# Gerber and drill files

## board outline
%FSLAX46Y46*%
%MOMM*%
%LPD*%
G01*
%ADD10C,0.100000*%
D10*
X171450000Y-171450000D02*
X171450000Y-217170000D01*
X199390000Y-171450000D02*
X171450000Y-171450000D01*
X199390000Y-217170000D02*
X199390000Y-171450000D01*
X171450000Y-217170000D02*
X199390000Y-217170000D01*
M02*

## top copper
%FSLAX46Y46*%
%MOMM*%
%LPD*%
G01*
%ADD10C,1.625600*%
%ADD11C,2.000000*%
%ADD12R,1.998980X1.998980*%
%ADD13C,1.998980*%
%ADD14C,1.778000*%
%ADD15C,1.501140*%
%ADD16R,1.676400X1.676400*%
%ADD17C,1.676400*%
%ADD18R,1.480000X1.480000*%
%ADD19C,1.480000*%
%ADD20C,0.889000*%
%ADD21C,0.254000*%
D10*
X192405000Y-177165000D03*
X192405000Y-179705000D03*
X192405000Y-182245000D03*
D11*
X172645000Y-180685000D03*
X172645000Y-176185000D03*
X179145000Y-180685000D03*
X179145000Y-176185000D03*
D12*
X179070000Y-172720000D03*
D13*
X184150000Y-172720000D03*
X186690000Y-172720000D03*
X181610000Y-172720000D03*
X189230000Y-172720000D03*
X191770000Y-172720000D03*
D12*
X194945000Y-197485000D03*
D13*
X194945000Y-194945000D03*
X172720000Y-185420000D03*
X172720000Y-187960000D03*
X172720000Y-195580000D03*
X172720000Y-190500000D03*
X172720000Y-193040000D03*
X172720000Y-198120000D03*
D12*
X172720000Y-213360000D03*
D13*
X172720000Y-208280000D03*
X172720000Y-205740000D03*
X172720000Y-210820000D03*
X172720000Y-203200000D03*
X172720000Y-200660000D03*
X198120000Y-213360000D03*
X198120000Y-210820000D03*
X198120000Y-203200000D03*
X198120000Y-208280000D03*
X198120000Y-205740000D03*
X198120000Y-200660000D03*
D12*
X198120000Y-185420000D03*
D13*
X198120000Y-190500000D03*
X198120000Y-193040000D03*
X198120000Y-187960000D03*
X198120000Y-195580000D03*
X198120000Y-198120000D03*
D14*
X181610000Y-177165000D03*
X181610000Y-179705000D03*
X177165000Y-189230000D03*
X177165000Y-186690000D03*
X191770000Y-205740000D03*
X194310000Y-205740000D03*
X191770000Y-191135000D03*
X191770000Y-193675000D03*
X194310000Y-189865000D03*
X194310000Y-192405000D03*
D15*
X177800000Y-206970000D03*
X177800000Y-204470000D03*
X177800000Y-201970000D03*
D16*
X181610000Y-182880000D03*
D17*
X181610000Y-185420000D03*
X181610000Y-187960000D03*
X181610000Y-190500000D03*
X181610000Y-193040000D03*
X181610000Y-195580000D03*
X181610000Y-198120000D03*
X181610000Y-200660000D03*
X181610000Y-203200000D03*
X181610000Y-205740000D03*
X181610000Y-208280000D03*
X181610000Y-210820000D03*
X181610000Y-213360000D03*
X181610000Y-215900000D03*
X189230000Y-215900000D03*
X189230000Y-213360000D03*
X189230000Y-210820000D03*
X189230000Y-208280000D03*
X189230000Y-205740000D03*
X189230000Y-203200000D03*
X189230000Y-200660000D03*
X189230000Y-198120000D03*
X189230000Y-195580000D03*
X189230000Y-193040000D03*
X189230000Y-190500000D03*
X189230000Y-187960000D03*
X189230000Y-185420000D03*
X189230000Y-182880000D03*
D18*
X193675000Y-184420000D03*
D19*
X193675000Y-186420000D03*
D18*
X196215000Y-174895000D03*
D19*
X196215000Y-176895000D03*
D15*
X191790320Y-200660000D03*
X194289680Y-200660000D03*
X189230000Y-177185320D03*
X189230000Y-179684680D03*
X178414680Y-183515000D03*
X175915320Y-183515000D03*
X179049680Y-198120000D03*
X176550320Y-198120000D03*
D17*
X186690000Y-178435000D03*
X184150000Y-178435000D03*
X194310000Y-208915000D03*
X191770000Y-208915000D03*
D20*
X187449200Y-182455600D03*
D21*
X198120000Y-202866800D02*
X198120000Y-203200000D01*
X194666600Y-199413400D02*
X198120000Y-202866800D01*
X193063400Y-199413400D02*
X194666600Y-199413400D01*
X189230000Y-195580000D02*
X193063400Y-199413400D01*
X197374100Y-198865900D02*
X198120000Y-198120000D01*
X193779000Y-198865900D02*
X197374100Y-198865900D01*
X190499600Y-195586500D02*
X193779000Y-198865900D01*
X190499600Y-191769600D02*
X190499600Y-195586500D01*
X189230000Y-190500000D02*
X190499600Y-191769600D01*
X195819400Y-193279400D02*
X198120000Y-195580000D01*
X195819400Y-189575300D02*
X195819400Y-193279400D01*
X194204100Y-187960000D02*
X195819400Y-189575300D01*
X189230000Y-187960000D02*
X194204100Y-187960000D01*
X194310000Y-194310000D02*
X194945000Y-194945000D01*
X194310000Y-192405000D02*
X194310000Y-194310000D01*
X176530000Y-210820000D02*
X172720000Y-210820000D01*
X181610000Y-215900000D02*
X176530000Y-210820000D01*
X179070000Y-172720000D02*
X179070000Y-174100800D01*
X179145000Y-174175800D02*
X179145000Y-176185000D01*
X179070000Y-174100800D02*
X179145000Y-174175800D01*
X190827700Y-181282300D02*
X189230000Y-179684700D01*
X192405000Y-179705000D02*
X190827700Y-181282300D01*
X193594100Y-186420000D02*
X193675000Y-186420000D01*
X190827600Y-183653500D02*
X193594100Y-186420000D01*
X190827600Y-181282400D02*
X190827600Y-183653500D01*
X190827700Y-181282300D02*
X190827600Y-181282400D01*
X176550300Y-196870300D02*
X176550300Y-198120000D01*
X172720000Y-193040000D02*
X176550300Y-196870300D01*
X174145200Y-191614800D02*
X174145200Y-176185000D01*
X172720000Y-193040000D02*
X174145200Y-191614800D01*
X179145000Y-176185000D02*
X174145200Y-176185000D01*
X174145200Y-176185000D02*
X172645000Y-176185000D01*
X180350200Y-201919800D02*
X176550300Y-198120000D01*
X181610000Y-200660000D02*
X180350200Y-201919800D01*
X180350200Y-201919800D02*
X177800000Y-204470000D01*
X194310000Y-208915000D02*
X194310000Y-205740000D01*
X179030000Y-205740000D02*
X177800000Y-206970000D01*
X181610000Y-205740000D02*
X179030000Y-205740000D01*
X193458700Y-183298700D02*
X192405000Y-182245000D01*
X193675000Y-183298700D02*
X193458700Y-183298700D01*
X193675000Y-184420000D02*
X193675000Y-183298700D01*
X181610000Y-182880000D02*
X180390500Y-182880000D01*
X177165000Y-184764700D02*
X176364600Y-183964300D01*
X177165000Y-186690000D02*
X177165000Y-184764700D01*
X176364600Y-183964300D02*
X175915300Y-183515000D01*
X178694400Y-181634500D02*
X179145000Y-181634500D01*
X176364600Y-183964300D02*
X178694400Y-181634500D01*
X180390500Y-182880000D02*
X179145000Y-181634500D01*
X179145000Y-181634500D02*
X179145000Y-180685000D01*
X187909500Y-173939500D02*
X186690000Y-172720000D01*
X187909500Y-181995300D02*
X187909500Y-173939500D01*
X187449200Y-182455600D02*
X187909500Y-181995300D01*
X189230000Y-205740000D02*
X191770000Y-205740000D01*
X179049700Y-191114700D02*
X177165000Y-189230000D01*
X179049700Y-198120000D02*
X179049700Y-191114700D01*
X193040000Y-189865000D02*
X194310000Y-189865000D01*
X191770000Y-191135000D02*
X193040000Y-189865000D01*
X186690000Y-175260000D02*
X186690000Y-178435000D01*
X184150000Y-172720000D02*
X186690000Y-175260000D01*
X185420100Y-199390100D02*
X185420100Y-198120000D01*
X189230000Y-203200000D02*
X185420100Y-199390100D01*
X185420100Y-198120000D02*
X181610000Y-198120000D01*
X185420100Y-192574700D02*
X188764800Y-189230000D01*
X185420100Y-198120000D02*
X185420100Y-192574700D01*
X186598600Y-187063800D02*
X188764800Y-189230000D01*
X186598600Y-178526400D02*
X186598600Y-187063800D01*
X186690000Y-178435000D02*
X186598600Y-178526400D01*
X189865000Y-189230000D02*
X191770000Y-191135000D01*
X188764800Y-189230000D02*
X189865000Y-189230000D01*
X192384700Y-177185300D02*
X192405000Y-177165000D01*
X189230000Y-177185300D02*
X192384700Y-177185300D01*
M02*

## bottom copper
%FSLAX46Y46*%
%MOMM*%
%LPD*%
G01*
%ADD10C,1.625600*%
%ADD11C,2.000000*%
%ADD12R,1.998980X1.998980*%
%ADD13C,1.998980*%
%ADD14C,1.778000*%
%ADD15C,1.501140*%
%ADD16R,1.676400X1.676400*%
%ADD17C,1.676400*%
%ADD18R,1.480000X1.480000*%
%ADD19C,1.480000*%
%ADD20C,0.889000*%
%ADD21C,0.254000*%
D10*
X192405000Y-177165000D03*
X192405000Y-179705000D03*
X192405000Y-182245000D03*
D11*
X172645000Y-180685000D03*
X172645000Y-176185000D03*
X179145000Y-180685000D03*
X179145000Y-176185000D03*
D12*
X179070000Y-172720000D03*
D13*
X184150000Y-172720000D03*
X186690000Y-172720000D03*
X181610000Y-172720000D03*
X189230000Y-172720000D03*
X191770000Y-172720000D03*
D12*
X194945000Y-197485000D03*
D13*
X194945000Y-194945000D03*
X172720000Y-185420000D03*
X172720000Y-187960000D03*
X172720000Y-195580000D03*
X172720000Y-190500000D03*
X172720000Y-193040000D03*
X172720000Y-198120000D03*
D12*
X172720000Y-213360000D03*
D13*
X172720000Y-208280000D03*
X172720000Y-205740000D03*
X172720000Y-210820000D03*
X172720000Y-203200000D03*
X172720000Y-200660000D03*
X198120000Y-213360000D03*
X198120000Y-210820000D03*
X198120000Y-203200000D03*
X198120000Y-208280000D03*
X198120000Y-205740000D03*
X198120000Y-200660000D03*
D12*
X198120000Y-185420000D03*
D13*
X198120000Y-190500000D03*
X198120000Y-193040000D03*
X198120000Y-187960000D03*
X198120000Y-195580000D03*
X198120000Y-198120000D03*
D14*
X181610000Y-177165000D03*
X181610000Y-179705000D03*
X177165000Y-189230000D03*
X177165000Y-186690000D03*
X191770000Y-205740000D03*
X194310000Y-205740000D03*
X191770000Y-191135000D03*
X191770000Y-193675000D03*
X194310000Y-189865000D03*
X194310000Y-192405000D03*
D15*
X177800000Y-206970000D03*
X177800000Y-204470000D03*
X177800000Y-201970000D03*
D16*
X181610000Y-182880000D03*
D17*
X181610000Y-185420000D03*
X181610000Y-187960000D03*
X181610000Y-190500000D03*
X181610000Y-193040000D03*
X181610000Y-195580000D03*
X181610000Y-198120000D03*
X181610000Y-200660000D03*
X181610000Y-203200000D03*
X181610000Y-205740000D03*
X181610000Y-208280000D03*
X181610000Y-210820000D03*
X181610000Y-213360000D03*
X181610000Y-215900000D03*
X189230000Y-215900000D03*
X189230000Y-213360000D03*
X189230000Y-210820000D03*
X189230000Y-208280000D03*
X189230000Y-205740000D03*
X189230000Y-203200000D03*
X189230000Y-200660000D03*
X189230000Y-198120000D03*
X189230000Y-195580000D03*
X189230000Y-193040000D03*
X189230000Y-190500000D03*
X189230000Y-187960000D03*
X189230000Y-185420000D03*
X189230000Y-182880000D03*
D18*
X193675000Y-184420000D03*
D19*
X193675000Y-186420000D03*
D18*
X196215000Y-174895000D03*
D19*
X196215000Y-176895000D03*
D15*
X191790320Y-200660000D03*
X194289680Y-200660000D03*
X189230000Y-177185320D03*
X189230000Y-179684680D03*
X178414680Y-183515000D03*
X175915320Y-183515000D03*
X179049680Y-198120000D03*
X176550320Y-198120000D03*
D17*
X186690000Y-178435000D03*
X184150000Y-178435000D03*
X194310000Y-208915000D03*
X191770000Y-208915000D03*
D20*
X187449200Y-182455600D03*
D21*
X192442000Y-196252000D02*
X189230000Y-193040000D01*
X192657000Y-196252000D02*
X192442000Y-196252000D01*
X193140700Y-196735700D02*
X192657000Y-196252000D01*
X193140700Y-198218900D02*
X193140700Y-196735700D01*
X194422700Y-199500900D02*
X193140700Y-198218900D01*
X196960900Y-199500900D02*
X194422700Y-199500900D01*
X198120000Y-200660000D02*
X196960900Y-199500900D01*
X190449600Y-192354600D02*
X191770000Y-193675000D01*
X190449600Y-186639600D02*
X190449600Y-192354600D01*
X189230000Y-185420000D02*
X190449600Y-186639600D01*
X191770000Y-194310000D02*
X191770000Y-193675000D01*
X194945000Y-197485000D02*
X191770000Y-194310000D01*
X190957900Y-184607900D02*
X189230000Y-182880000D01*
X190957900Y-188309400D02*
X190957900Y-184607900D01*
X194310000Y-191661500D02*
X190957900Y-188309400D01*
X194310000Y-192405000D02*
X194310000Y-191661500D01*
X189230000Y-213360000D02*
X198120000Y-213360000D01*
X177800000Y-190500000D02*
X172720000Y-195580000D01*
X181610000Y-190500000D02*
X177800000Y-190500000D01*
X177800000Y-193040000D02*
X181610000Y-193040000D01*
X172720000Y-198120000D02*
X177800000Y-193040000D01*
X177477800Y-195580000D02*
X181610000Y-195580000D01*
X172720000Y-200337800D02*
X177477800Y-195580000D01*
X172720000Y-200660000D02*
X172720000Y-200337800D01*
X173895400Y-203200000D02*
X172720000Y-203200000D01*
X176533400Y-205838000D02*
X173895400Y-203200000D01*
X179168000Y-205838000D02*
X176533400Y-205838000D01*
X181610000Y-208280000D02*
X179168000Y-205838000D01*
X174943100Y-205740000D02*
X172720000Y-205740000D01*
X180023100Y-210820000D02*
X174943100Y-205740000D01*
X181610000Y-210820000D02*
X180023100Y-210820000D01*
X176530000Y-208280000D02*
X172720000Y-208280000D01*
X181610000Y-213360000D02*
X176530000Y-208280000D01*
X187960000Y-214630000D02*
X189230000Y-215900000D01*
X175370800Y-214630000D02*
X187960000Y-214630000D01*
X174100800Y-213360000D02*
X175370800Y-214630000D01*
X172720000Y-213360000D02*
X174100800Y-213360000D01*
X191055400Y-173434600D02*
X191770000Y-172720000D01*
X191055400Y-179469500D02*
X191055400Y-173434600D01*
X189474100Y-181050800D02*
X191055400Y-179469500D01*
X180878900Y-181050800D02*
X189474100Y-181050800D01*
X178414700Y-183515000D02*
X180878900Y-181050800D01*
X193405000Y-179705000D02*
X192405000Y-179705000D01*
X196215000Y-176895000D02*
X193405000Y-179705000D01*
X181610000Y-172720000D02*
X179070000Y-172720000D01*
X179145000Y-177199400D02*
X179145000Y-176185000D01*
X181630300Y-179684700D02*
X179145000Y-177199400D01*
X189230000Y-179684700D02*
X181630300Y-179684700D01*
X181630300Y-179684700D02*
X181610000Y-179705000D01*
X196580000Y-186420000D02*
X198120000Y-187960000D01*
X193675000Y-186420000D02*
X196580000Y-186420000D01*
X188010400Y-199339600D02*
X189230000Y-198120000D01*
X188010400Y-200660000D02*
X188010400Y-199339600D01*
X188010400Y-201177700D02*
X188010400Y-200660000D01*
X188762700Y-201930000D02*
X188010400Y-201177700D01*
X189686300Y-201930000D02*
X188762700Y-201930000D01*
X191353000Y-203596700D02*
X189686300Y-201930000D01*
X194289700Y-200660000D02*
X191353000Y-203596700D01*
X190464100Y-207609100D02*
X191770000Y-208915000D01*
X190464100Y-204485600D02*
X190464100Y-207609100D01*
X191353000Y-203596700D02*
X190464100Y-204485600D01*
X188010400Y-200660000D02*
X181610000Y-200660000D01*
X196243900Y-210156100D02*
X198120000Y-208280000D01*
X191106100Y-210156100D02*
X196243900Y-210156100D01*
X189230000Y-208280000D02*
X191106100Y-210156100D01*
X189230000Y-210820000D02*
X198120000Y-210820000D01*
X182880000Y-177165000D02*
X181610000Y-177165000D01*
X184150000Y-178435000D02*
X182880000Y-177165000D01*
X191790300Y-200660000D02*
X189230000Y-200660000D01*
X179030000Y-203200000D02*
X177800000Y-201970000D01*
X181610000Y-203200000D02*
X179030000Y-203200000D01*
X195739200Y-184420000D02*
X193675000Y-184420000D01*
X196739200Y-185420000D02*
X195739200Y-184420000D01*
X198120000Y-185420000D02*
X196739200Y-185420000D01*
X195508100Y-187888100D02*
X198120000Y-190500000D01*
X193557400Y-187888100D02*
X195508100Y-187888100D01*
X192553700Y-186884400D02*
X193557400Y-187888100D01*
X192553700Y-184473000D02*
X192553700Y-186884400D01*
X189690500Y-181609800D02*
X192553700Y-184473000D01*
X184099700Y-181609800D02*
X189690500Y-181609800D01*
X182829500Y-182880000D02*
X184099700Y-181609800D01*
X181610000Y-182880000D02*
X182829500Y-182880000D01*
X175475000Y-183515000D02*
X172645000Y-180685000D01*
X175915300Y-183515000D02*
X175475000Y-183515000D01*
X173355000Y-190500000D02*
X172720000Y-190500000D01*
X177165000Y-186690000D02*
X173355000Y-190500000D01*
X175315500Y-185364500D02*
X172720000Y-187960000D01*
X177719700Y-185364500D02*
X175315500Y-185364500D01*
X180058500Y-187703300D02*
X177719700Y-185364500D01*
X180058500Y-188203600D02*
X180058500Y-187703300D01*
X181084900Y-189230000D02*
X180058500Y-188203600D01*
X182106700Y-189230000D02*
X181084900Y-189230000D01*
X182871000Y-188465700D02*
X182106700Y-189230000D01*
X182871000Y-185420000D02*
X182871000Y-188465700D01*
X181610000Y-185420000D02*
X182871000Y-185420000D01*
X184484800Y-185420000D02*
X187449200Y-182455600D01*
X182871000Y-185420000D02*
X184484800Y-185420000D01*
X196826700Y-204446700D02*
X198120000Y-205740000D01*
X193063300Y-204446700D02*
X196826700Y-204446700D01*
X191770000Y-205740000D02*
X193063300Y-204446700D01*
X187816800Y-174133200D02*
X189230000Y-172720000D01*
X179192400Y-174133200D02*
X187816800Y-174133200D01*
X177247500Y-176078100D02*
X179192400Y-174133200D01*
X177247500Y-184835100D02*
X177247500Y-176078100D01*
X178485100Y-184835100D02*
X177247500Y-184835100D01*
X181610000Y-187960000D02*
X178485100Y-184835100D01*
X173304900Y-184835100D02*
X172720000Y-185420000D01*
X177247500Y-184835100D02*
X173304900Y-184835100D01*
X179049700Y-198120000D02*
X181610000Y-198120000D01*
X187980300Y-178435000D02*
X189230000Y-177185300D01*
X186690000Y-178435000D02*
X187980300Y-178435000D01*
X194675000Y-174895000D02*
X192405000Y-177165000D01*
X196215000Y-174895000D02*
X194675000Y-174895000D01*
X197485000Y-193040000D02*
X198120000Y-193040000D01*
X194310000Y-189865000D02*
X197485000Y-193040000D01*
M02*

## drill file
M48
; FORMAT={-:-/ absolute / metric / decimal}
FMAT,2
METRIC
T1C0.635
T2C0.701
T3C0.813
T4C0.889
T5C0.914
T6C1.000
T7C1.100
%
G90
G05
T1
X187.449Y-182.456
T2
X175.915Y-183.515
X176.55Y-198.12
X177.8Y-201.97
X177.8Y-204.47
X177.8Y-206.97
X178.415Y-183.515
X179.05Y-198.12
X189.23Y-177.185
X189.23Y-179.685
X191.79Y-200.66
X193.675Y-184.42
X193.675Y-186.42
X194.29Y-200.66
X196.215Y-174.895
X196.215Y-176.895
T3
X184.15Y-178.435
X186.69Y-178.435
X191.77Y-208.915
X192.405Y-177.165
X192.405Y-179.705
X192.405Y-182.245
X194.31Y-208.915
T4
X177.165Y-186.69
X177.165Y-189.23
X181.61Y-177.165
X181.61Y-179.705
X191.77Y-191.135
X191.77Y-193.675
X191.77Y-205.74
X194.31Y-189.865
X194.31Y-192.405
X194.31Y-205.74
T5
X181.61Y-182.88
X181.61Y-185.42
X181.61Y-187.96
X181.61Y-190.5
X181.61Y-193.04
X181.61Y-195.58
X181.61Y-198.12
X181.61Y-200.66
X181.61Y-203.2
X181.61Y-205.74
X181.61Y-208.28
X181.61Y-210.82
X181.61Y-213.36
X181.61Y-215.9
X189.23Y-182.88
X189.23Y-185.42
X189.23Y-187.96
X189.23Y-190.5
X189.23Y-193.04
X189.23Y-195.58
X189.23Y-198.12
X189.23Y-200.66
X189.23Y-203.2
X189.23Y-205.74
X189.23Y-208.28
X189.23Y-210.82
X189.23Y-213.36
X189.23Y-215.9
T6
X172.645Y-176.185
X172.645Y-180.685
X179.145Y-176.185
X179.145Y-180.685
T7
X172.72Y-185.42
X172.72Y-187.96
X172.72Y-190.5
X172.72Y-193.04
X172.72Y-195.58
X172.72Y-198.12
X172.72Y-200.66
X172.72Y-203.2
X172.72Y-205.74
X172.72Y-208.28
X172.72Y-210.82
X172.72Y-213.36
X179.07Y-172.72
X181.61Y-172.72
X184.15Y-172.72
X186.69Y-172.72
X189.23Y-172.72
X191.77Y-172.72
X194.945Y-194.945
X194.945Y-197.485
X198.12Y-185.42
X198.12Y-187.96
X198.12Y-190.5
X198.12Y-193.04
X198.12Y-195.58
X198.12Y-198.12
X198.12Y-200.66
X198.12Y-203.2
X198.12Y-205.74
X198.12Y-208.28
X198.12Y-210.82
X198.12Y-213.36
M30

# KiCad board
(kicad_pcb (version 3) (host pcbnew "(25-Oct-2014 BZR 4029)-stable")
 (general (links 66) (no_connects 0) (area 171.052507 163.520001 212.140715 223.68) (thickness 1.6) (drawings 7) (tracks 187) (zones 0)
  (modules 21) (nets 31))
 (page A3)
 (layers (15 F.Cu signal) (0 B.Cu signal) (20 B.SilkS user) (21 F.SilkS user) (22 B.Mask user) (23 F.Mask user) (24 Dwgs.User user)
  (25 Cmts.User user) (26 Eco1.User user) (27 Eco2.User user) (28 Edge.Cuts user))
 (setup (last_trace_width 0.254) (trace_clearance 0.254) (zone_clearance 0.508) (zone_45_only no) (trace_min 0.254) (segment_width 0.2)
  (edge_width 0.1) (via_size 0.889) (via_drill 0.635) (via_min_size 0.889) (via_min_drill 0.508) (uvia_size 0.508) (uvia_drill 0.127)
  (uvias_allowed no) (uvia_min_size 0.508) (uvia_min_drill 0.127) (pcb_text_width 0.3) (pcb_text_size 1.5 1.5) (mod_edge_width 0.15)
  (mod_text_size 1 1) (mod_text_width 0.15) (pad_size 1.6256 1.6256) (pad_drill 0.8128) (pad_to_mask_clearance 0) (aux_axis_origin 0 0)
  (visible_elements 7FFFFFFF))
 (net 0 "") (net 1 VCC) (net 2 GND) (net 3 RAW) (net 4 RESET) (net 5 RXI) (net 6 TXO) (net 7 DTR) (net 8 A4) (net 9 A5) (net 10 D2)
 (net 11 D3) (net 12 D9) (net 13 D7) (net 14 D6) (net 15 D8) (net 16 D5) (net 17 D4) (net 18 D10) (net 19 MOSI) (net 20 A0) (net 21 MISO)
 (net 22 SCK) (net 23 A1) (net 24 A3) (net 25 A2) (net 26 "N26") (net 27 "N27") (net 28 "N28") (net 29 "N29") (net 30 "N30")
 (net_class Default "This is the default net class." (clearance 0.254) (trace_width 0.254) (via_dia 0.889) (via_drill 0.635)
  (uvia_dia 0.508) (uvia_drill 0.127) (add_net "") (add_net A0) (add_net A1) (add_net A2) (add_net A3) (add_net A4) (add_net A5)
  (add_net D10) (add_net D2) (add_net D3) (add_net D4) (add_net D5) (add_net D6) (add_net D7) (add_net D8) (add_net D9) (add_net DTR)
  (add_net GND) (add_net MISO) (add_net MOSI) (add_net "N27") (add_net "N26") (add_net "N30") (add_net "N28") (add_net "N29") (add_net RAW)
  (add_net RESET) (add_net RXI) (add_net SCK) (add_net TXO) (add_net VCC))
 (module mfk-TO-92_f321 (layer F.Cu) (at 192.405 179.705 270)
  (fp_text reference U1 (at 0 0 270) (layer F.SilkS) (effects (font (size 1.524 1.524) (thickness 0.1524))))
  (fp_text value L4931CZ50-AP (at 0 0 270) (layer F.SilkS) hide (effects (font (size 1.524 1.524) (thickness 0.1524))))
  (pad 3 thru_hole circle (at -2.54 0 270) (size 1.6256 1.6256) (drill 0.8128) (layers *.Cu *.Mask F.SilkS) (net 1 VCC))
  (pad 2 thru_hole circle (at 0 0 270) (size 1.6256 1.6256) (drill 0.8128) (layers *.Cu *.Mask F.SilkS) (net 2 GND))
  (pad 1 thru_hole circle (at 2.54 0 270) (size 1.6256 1.6256) (drill 0.8128) (layers *.Cu *.Mask F.SilkS) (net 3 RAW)))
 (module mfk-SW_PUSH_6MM (layer F.Cu) (at 175.895 178.435 180)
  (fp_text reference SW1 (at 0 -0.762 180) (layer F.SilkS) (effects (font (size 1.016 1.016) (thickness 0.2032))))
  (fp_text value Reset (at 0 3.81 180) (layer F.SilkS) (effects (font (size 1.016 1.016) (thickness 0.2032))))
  (pad 1 thru_hole circle (at 3.25 -2.25 180) (size 2 2) (drill 1) (layers *.Cu *.Mask F.SilkS) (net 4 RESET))
  (pad 2 thru_hole circle (at 3.25 2.25 180) (size 2 2) (drill 1) (layers *.Cu *.Mask F.SilkS) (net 2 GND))
  (pad 1 thru_hole circle (at -3.25 -2.25 180) (size 2 2) (drill 1) (layers *.Cu *.Mask F.SilkS) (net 4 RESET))
  (pad 2 thru_hole circle (at -3.25 2.25 180) (size 2 2) (drill 1) (layers *.Cu *.Mask F.SilkS) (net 2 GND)))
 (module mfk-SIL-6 (layer F.Cu) (at 185.42 172.72)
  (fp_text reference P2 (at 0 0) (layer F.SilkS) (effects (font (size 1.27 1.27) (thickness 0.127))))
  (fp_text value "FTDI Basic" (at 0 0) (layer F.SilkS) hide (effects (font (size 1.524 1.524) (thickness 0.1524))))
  (pad 1 thru_hole rect (at -6.35 0) (size 1.99898 1.99898) (drill 1.09982) (layers *.Cu *.Mask F.SilkS) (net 2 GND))
  (pad 3 thru_hole circle (at -1.27 0) (size 1.99898 1.99898) (drill 1.09982) (layers *.Cu *.Mask F.SilkS) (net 1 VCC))
  (pad 4 thru_hole circle (at 1.27 0) (size 1.99898 1.99898) (drill 1.09982) (layers *.Cu *.Mask F.SilkS) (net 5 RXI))
  (pad 2 thru_hole circle (at -3.81 0) (size 1.99898 1.99898) (drill 1.09982) (layers *.Cu *.Mask F.SilkS) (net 2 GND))
  (pad 5 thru_hole circle (at 3.81 0) (size 1.99898 1.99898) (drill 1.09982) (layers *.Cu *.Mask F.SilkS) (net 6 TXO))
  (pad 6 thru_hole circle (at 6.35 0) (size 1.99898 1.99898) (drill 1.09982) (layers *.Cu *.Mask F.SilkS) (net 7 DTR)))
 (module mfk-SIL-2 (layer F.Cu) (at 194.945 196.215 90)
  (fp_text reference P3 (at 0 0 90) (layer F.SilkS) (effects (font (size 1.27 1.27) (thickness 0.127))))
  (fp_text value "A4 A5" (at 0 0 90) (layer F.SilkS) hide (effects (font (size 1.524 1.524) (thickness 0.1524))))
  (pad 1 thru_hole rect (at -1.27 0 90) (size 1.99898 1.99898) (drill 1.09982) (layers *.Cu *.Mask F.SilkS) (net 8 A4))
  (pad 2 thru_hole circle (at 1.27 0 90) (size 1.99898 1.99898) (drill 1.09982) (layers *.Cu *.Mask F.SilkS) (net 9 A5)))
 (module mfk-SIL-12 (layer F.Cu) (at 172.72 199.39 90)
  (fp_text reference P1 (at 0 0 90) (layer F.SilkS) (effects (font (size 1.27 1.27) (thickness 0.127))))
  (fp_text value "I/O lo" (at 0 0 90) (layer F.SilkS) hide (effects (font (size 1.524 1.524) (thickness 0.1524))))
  (pad 12 thru_hole circle (at 13.97 0 90) (size 1.99898 1.99898) (drill 1.09982) (layers *.Cu *.Mask F.SilkS) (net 6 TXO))
  (pad 11 thru_hole circle (at 11.43 0 90) (size 1.99898 1.99898) (drill 1.09982) (layers *.Cu *.Mask F.SilkS) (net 5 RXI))
  (pad 8 thru_hole circle (at 3.81 0 90) (size 1.99898 1.99898) (drill 1.09982) (layers *.Cu *.Mask F.SilkS) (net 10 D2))
  (pad 10 thru_hole circle (at 8.89 0 90) (size 1.99898 1.99898) (drill 1.09982) (layers *.Cu *.Mask F.SilkS) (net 4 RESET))
  (pad 9 thru_hole circle (at 6.35 0 90) (size 1.99898 1.99898) (drill 1.09982) (layers *.Cu *.Mask F.SilkS) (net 2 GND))
  (pad 7 thru_hole circle (at 1.27 0 90) (size 1.99898 1.99898) (drill 1.09982) (layers *.Cu *.Mask F.SilkS) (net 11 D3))
  (pad 1 thru_hole rect (at -13.97 0 90) (size 1.99898 1.99898) (drill 1.09982) (layers *.Cu *.Mask F.SilkS) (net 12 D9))
  (pad 3 thru_hole circle (at -8.89 0 90) (size 1.99898 1.99898) (drill 1.09982) (layers *.Cu *.Mask F.SilkS) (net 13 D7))
  (pad 4 thru_hole circle (at -6.35 0 90) (size 1.99898 1.99898) (drill 1.09982) (layers *.Cu *.Mask F.SilkS) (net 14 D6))
  (pad 2 thru_hole circle (at -11.43 0 90) (size 1.99898 1.99898) (drill 1.09982) (layers *.Cu *.Mask F.SilkS) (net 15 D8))
  (pad 5 thru_hole circle (at -3.81 0 90) (size 1.99898 1.99898) (drill 1.09982) (layers *.Cu *.Mask F.SilkS) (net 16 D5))
  (pad 6 thru_hole circle (at -1.27 0 90) (size 1.99898 1.99898) (drill 1.09982) (layers *.Cu *.Mask F.SilkS) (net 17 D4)))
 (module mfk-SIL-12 (layer F.Cu) (at 198.12 199.39 270)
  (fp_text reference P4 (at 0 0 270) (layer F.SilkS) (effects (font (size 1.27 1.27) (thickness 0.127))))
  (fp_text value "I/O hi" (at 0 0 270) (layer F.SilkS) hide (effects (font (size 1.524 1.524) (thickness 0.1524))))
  (pad 12 thru_hole circle (at 13.97 0 270) (size 1.99898 1.99898) (drill 1.09982) (layers *.Cu *.Mask F.SilkS) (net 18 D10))
  (pad 11 thru_hole circle (at 11.43 0 270) (size 1.99898 1.99898) (drill 1.09982) (layers *.Cu *.Mask F.SilkS) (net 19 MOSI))
  (pad 8 thru_hole circle (at 3.81 0 270) (size 1.99898 1.99898) (drill 1.09982) (layers *.Cu *.Mask F.SilkS) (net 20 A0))
  (pad 10 thru_hole circle (at 8.89 0 270) (size 1.99898 1.99898) (drill 1.09982) (layers *.Cu *.Mask F.SilkS) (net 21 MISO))
  (pad 9 thru_hole circle (at 6.35 0 270) (size 1.99898 1.99898) (drill 1.09982) (layers *.Cu *.Mask F.SilkS) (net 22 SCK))
  (pad 7 thru_hole circle (at 1.27 0 270) (size 1.99898 1.99898) (drill 1.09982) (layers *.Cu *.Mask F.SilkS) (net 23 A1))
  (pad 1 thru_hole rect (at -13.97 0 270) (size 1.99898 1.99898) (drill 1.09982) (layers *.Cu *.Mask F.SilkS) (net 3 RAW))
  (pad 3 thru_hole circle (at -8.89 0 270) (size 1.99898 1.99898) (drill 1.09982) (layers *.Cu *.Mask F.SilkS) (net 4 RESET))
  (pad 4 thru_hole circle (at -6.35 0 270) (size 1.99898 1.99898) (drill 1.09982) (layers *.Cu *.Mask F.SilkS) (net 1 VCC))
  (pad 2 thru_hole circle (at -11.43 0 270) (size 1.99898 1.99898) (drill 1.09982) (layers *.Cu *.Mask F.SilkS) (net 2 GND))
  (pad 5 thru_hole circle (at -3.81 0 270) (size 1.99898 1.99898) (drill 1.09982) (layers *.Cu *.Mask F.SilkS) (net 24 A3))
  (pad 6 thru_hole circle (at -1.27 0 270) (size 1.99898 1.99898) (drill 1.09982) (layers *.Cu *.Mask F.SilkS) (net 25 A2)))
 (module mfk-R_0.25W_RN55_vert (layer F.Cu) (at 181.61 178.435 270)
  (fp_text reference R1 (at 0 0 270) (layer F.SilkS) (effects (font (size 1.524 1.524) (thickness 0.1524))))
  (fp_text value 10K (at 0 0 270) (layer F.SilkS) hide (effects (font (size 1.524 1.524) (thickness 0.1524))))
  (pad 1 thru_hole circle (at -1.27 0 270) (size 1.778 1.778) (drill 0.889) (layers *.Cu *.Mask F.SilkS) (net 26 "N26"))
  (pad 2 thru_hole circle (at 1.27 0 270) (size 1.778 1.778) (drill 0.889) (layers *.Cu *.Mask F.SilkS) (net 2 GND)))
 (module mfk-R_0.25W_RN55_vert (layer F.Cu) (at 177.165 187.96 90)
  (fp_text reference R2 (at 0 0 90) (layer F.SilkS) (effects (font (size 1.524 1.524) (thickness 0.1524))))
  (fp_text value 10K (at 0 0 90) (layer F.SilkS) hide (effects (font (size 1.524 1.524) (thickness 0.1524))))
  (pad 1 thru_hole circle (at -1.27 0 90) (size 1.778 1.778) (drill 0.889) (layers *.Cu *.Mask F.SilkS) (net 1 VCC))
  (pad 2 thru_hole circle (at 1.27 0 90) (size 1.778 1.778) (drill 0.889) (layers *.Cu *.Mask F.SilkS) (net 4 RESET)))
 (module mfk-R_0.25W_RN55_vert (layer F.Cu) (at 193.04 205.74)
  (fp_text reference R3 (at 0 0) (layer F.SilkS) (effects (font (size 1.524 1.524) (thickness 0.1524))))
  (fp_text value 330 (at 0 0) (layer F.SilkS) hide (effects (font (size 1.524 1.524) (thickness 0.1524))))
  (pad 1 thru_hole circle (at -1.27 0) (size 1.778 1.778) (drill 0.889) (layers *.Cu *.Mask F.SilkS) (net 22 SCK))
  (pad 2 thru_hole circle (at 1.27 0) (size 1.778 1.778) (drill 0.889) (layers *.Cu *.Mask F.SilkS) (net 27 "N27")))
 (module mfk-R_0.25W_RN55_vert (layer F.Cu) (at 191.77 192.405 270)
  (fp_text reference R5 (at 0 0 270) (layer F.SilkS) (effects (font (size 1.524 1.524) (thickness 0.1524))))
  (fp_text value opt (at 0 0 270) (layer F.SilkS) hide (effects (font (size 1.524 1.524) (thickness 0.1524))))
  (pad 1 thru_hole circle (at -1.27 0 270) (size 1.778 1.778) (drill 0.889) (layers *.Cu *.Mask F.SilkS) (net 1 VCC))
  (pad 2 thru_hole circle (at 1.27 0 270) (size 1.778 1.778) (drill 0.889) (layers *.Cu *.Mask F.SilkS) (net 8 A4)))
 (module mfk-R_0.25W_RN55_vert (layer F.Cu) (at 194.31 191.135 270)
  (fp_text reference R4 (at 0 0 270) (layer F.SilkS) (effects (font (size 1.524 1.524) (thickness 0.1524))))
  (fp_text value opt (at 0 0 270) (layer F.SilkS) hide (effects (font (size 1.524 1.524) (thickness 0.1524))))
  (pad 1 thru_hole circle (at -1.27 0 270) (size 1.778 1.778) (drill 0.889) (layers *.Cu *.Mask F.SilkS) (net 1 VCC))
  (pad 2 thru_hole circle (at 1.27 0 270) (size 1.778 1.778) (drill 0.889) (layers *.Cu *.Mask F.SilkS) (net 9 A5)))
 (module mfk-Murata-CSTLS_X (layer F.Cu) (at 177.8 204.47 90)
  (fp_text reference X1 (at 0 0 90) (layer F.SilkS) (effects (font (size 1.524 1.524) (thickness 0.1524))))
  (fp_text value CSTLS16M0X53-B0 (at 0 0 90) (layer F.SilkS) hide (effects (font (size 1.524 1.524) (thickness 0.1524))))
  (pad 1 thru_hole circle (at -2.5 0 90) (size 1.50114 1.50114) (drill 0.70104) (layers *.Cu *.Mask F.SilkS) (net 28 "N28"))
  (pad 3 thru_hole circle (at 0 0 90) (size 1.50114 1.50114) (drill 0.70104) (layers *.Cu *.Mask F.SilkS) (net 2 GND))
  (pad 2 thru_hole circle (at 2.5 0 90) (size 1.50114 1.50114) (drill 0.70104) (layers *.Cu *.Mask F.SilkS) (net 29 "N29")))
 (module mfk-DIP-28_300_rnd (layer F.Cu) (at 185.42 199.39)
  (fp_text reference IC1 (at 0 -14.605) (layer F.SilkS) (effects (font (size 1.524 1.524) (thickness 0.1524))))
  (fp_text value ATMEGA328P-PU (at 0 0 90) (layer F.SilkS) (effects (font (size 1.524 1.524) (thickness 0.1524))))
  (pad 1 thru_hole rect (at -3.81 -16.51) (size 1.6764 1.6764) (drill 0.9144) (layers *.Cu *.Mask F.SilkS) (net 4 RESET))
  (pad 2 thru_hole circle (at -3.81 -13.97) (size 1.6764 1.6764) (drill 0.9144) (layers *.Cu *.Mask F.SilkS) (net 5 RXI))
  (pad 3 thru_hole circle (at -3.81 -11.43) (size 1.6764 1.6764) (drill 0.9144) (layers *.Cu *.Mask F.SilkS) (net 6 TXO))
  (pad 4 thru_hole circle (at -3.81 -8.89) (size 1.6764 1.6764) (drill 0.9144) (layers *.Cu *.Mask F.SilkS) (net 10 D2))
  (pad 5 thru_hole circle (at -3.81 -6.35) (size 1.6764 1.6764) (drill 0.9144) (layers *.Cu *.Mask F.SilkS) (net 11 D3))
  (pad 6 thru_hole circle (at -3.81 -3.81) (size 1.6764 1.6764) (drill 0.9144) (layers *.Cu *.Mask F.SilkS) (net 17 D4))
  (pad 7 thru_hole circle (at -3.81 -1.27) (size 1.6764 1.6764) (drill 0.9144) (layers *.Cu *.Mask F.SilkS) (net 1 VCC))
  (pad 8 thru_hole circle (at -3.81 1.27) (size 1.6764 1.6764) (drill 0.9144) (layers *.Cu *.Mask F.SilkS) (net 2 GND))
  (pad 9 thru_hole circle (at -3.81 3.81) (size 1.6764 1.6764) (drill 0.9144) (layers *.Cu *.Mask F.SilkS) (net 29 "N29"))
  (pad 10 thru_hole circle (at -3.81 6.35) (size 1.6764 1.6764) (drill 0.9144) (layers *.Cu *.Mask F.SilkS) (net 28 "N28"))
  (pad 11 thru_hole circle (at -3.81 8.89) (size 1.6764 1.6764) (drill 0.9144) (layers *.Cu *.Mask F.SilkS) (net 16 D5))
  (pad 12 thru_hole circle (at -3.81 11.43) (size 1.6764 1.6764) (drill 0.9144) (layers *.Cu *.Mask F.SilkS) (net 14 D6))
  (pad 13 thru_hole circle (at -3.81 13.97) (size 1.6764 1.6764) (drill 0.9144) (layers *.Cu *.Mask F.SilkS) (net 13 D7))
  (pad 14 thru_hole circle (at -3.81 16.51) (size 1.6764 1.6764) (drill 0.9144) (layers *.Cu *.Mask F.SilkS) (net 15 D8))
  (pad 15 thru_hole circle (at 3.81 16.51) (size 1.6764 1.6764) (drill 0.9144) (layers *.Cu *.Mask F.SilkS) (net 12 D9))
  (pad 16 thru_hole circle (at 3.81 13.97) (size 1.6764 1.6764) (drill 0.9144) (layers *.Cu *.Mask F.SilkS) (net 18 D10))
  (pad 17 thru_hole circle (at 3.81 11.43) (size 1.6764 1.6764) (drill 0.9144) (layers *.Cu *.Mask F.SilkS) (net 19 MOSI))
  (pad 18 thru_hole circle (at 3.81 8.89) (size 1.6764 1.6764) (drill 0.9144) (layers *.Cu *.Mask F.SilkS) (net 21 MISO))
  (pad 19 thru_hole circle (at 3.81 6.35) (size 1.6764 1.6764) (drill 0.9144) (layers *.Cu *.Mask F.SilkS) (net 22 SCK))
  (pad 20 thru_hole circle (at 3.81 3.81) (size 1.6764 1.6764) (drill 0.9144) (layers *.Cu *.Mask F.SilkS) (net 1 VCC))
  (pad 21 thru_hole circle (at 3.81 1.27) (size 1.6764 1.6764) (drill 0.9144) (layers *.Cu *.Mask F.SilkS) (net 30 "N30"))
  (pad 22 thru_hole circle (at 3.81 -1.27) (size 1.6764 1.6764) (drill 0.9144) (layers *.Cu *.Mask F.SilkS) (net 2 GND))
  (pad 23 thru_hole circle (at 3.81 -3.81) (size 1.6764 1.6764) (drill 0.9144) (layers *.Cu *.Mask F.SilkS) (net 20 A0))
  (pad 24 thru_hole circle (at 3.81 -6.35) (size 1.6764 1.6764) (drill 0.9144) (layers *.Cu *.Mask F.SilkS) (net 23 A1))
  (pad 25 thru_hole circle (at 3.81 -8.89) (size 1.6764 1.6764) (drill 0.9144) (layers *.Cu *.Mask F.SilkS) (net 25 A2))
  (pad 26 thru_hole circle (at 3.81 -11.43) (size 1.6764 1.6764) (drill 0.9144) (layers *.Cu *.Mask F.SilkS) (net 24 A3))
  (pad 27 thru_hole circle (at 3.81 -13.97) (size 1.6764 1.6764) (drill 0.9144) (layers *.Cu *.Mask F.SilkS) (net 8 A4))
  (pad 28 thru_hole circle (at 3.81 -16.51) (size 1.6764 1.6764) (drill 0.9144) (layers *.Cu *.Mask F.SilkS) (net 9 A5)))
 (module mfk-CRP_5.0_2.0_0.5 (layer F.Cu) (at 193.675 185.42 270)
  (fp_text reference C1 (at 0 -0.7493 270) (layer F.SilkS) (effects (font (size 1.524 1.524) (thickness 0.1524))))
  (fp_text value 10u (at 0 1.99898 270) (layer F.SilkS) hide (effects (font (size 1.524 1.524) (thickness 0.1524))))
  (pad 1 thru_hole rect (at -1 0 270) (size 1.48 1.48) (drill 0.70104) (layers *.Cu *.Mask F.SilkS) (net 3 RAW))
  (pad 2 thru_hole circle (at 1 0 270) (size 1.48 1.48) (drill 0.70104) (layers *.Cu *.Mask F.SilkS) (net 2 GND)))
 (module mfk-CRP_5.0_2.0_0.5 (layer F.Cu) (at 196.215 175.895 270)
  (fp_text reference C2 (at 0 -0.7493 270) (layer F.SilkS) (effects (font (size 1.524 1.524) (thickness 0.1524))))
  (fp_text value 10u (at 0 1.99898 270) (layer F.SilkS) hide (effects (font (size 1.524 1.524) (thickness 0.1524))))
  (pad 1 thru_hole rect (at -1 0 270) (size 1.48 1.48) (drill 0.70104) (layers *.Cu *.Mask F.SilkS) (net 1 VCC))
  (pad 2 thru_hole circle (at 1 0 270) (size 1.48 1.48) (drill 0.70104) (layers *.Cu *.Mask F.SilkS) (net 2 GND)))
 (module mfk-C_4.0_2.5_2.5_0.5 (layer F.Cu) (at 193.04 200.66)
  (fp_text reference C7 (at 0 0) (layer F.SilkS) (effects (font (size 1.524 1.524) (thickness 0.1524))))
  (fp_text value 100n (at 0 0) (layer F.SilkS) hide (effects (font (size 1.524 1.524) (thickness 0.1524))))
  (pad 1 thru_hole circle (at -1.24968 0) (size 1.50114 1.50114) (drill 0.70104) (layers *.Cu *.Mask F.SilkS) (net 30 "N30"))
  (pad 2 thru_hole circle (at 1.24968 0) (size 1.50114 1.50114) (drill 0.70104) (layers *.Cu *.Mask F.SilkS) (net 2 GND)))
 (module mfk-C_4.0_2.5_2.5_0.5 (layer F.Cu) (at 189.23 178.435 270)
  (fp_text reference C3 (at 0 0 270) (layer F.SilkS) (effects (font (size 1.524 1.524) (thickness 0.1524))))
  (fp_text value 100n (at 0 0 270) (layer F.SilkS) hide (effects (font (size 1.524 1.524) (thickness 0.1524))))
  (pad 1 thru_hole circle (at -1.24968 0 270) (size 1.50114 1.50114) (drill 0.70104) (layers *.Cu *.Mask F.SilkS) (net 1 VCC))
  (pad 2 thru_hole circle (at 1.24968 0 270) (size 1.50114 1.50114) (drill 0.70104) (layers *.Cu *.Mask F.SilkS) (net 2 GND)))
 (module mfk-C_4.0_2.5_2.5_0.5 (layer F.Cu) (at 177.165 183.515 180)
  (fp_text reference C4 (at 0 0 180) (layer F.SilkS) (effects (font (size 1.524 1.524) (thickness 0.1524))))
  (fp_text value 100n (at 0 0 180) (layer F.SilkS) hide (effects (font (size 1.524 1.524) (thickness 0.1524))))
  (pad 1 thru_hole circle (at -1.24968 0 180) (size 1.50114 1.50114) (drill 0.70104) (layers *.Cu *.Mask F.SilkS) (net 7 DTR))
  (pad 2 thru_hole circle (at 1.24968 0 180) (size 1.50114 1.50114) (drill 0.70104) (layers *.Cu *.Mask F.SilkS) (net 4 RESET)))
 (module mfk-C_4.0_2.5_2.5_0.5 (layer F.Cu) (at 177.8 198.12 180)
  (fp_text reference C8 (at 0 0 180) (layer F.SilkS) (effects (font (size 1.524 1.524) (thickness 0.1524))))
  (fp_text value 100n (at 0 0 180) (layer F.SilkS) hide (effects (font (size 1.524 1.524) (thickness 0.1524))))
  (pad 1 thru_hole circle (at -1.24968 0 180) (size 1.50114 1.50114) (drill 0.70104) (layers *.Cu *.Mask F.SilkS) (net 1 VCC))
  (pad 2 thru_hole circle (at 1.24968 0 180) (size 1.50114 1.50114) (drill 0.70104) (layers *.Cu *.Mask F.SilkS) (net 2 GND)))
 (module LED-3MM (layer F.Cu) (at 185.42 178.435 180)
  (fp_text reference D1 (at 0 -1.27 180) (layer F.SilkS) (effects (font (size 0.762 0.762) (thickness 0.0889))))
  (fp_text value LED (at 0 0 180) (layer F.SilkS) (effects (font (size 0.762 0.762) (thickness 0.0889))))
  (pad 1 thru_hole circle (at -1.27 0 180) (size 1.6764 1.6764) (drill 0.8128) (layers *.Cu *.Mask F.SilkS) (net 1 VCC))
  (pad 2 thru_hole circle (at 1.27 0 180) (size 1.6764 1.6764) (drill 0.8128) (layers *.Cu *.Mask F.SilkS) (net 26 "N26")))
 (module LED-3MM (layer F.Cu) (at 193.04 208.915 180)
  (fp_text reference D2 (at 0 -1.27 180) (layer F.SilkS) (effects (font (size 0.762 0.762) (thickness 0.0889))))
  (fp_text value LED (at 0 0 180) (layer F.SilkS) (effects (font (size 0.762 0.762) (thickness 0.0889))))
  (pad 1 thru_hole circle (at -1.27 0 180) (size 1.6764 1.6764) (drill 0.8128) (layers *.Cu *.Mask F.SilkS) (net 27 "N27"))
  (pad 2 thru_hole circle (at 1.27 0 180) (size 1.6764 1.6764) (drill 0.8128) (layers *.Cu *.Mask F.SilkS) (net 2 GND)))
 (gr_line (start 171.45 171.45) (end 171.45 217.17) (angle 90) (layer Edge.Cuts) (width 0.1))
 (gr_line (start 199.39 171.45) (end 171.45 171.45) (angle 90) (layer Edge.Cuts) (width 0.1))
 (gr_line (start 199.39 217.17) (end 199.39 171.45) (angle 90) (layer Edge.Cuts) (width 0.1))
 (gr_line (start 171.45 217.17) (end 199.39 217.17) (angle 90) (layer Edge.Cuts) (width 0.1))
 (segment (start 198.12 202.8668) (end 198.12 203.2) (width 0.254) (layer F.Cu) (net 20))
 (segment (start 194.6666 199.4134) (end 198.12 202.8668) (width 0.254) (layer F.Cu) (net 20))
 (segment (start 193.0634 199.4134) (end 194.6666 199.4134) (width 0.254) (layer F.Cu) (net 20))
 (segment (start 189.23 195.58) (end 193.0634 199.4134) (width 0.254) (layer F.Cu) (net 20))
 (segment (start 192.442 196.252) (end 189.23 193.04) (width 0.254) (layer B.Cu) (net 23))
 (segment (start 192.657 196.252) (end 192.442 196.252) (width 0.254) (layer B.Cu) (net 23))
 (segment (start 193.1407 196.7357) (end 192.657 196.252) (width 0.254) (layer B.Cu) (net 23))
 (segment (start 193.1407 198.2189) (end 193.1407 196.7357) (width 0.254) (layer B.Cu) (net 23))
 (segment (start 194.4227 199.5009) (end 193.1407 198.2189) (width 0.254) (layer B.Cu) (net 23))
 (segment (start 196.9609 199.5009) (end 194.4227 199.5009) (width 0.254) (layer B.Cu) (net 23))
 (segment (start 198.12 200.66) (end 196.9609 199.5009) (width 0.254) (layer B.Cu) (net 23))
 (segment (start 197.3741 198.8659) (end 198.12 198.12) (width 0.254) (layer F.Cu) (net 25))
 (segment (start 193.779 198.8659) (end 197.3741 198.8659) (width 0.254) (layer F.Cu) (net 25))
 (segment (start 190.4996 195.5865) (end 193.779 198.8659) (width 0.254) (layer F.Cu) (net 25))
 (segment (start 190.4996 191.7696) (end 190.4996 195.5865) (width 0.254) (layer F.Cu) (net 25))
 (segment (start 189.23 190.5) (end 190.4996 191.7696) (width 0.254) (layer F.Cu) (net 25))
 (segment (start 195.8194 193.2794) (end 198.12 195.58) (width 0.254) (layer F.Cu) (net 24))
 (segment (start 195.8194 189.5753) (end 195.8194 193.2794) (width 0.254) (layer F.Cu) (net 24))
 (segment (start 194.2041 187.96) (end 195.8194 189.5753) (width 0.254) (layer F.Cu) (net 24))
 (segment (start 189.23 187.96) (end 194.2041 187.96) (width 0.254) (layer F.Cu) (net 24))
 (segment (start 190.4496 192.3546) (end 191.77 193.675) (width 0.254) (layer B.Cu) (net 8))
 (segment (start 190.4496 186.6396) (end 190.4496 192.3546) (width 0.254) (layer B.Cu) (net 8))
 (segment (start 189.23 185.42) (end 190.4496 186.6396) (width 0.254) (layer B.Cu) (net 8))
 (segment (start 191.77 194.31) (end 191.77 193.675) (width 0.254) (layer B.Cu) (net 8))
 (segment (start 194.945 197.485) (end 191.77 194.31) (width 0.254) (layer B.Cu) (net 8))
 (segment (start 190.9579 184.6079) (end 189.23 182.88) (width 0.254) (layer B.Cu) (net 9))
 (segment (start 190.9579 188.3094) (end 190.9579 184.6079) (width 0.254) (layer B.Cu) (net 9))
 (segment (start 194.31 191.6615) (end 190.9579 188.3094) (width 0.254) (layer B.Cu) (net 9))
 (segment (start 194.31 192.405) (end 194.31 191.6615) (width 0.254) (layer B.Cu) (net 9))
 (segment (start 194.31 194.31) (end 194.945 194.945) (width 0.254) (layer F.Cu) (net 9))
 (segment (start 194.31 192.405) (end 194.31 194.31) (width 0.254) (layer F.Cu) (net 9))
 (segment (start 189.23 213.36) (end 198.12 213.36) (width 0.254) (layer B.Cu) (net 18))
 (segment (start 177.8 190.5) (end 172.72 195.58) (width 0.254) (layer B.Cu) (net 10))
 (segment (start 181.61 190.5) (end 177.8 190.5) (width 0.254) (layer B.Cu) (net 10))
 (segment (start 177.8 193.04) (end 181.61 193.04) (width 0.254) (layer B.Cu) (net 11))
 (segment (start 172.72 198.12) (end 177.8 193.04) (width 0.254) (layer B.Cu) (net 11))
 (segment (start 177.4778 195.58) (end 181.61 195.58) (width 0.254) (layer B.Cu) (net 17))
 (segment (start 172.72 200.3378) (end 177.4778 195.58) (width 0.254) (layer B.Cu) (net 17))
 (segment (start 172.72 200.66) (end 172.72 200.3378) (width 0.254) (layer B.Cu) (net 17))
 (segment (start 173.8954 203.2) (end 172.72 203.2) (width 0.254) (layer B.Cu) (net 16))
 (segment (start 176.5334 205.838) (end 173.8954 203.2) (width 0.254) (layer B.Cu) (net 16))
 (segment (start 179.168 205.838) (end 176.5334 205.838) (width 0.254) (layer B.Cu) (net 16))
 (segment (start 181.61 208.28) (end 179.168 205.838) (width 0.254) (layer B.Cu) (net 16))
 (segment (start 174.9431 205.74) (end 172.72 205.74) (width 0.254) (layer B.Cu) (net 14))
 (segment (start 180.0231 210.82) (end 174.9431 205.74) (width 0.254) (layer B.Cu) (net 14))
 (segment (start 181.61 210.82) (end 180.0231 210.82) (width 0.254) (layer B.Cu) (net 14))
 (segment (start 176.53 208.28) (end 172.72 208.28) (width 0.254) (layer B.Cu) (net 13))
 (segment (start 181.61 213.36) (end 176.53 208.28) (width 0.254) (layer B.Cu) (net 13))
 (segment (start 176.53 210.82) (end 172.72 210.82) (width 0.254) (layer F.Cu) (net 15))
 (segment (start 181.61 215.9) (end 176.53 210.82) (width 0.254) (layer F.Cu) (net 15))
 (segment (start 187.96 214.63) (end 189.23 215.9) (width 0.254) (layer B.Cu) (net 12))
 (segment (start 175.3708 214.63) (end 187.96 214.63) (width 0.254) (layer B.Cu) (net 12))
 (segment (start 174.1008 213.36) (end 175.3708 214.63) (width 0.254) (layer B.Cu) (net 12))
 (segment (start 172.72 213.36) (end 174.1008 213.36) (width 0.254) (layer B.Cu) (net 12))
 (segment (start 191.0554 173.4346) (end 191.77 172.72) (width 0.254) (layer B.Cu) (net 7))
 (segment (start 191.0554 179.4695) (end 191.0554 173.4346) (width 0.254) (layer B.Cu) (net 7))
 (segment (start 189.4741 181.0508) (end 191.0554 179.4695) (width 0.254) (layer B.Cu) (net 7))
 (segment (start 180.8789 181.0508) (end 189.4741 181.0508) (width 0.254) (layer B.Cu) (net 7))
 (segment (start 178.4147 183.515) (end 180.8789 181.0508) (width 0.254) (layer B.Cu) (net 7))
 (segment (start 193.405 179.705) (end 192.405 179.705) (width 0.254) (layer B.Cu) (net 2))
 (segment (start 196.215 176.895) (end 193.405 179.705) (width 0.254) (layer B.Cu) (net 2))
 (segment (start 179.07 172.72) (end 179.07 174.1008) (width 0.254) (layer F.Cu) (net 2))
 (segment (start 181.61 172.72) (end 179.07 172.72) (width 0.254) (layer B.Cu) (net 2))
 (segment (start 179.145 177.1994) (end 179.145 176.185) (width 0.254) (layer B.Cu) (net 2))
 (segment (start 181.6303 179.6847) (end 179.145 177.1994) (width 0.254) (layer B.Cu) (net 2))
 (segment (start 189.23 179.6847) (end 181.6303 179.6847) (width 0.254) (layer B.Cu) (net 2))
 (segment (start 181.6303 179.6847) (end 181.61 179.705) (width 0.254) (layer B.Cu) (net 2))
 (segment (start 179.145 174.1758) (end 179.145 176.185) (width 0.254) (layer F.Cu) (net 2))
 (segment (start 179.07 174.1008) (end 179.145 174.1758) (width 0.254) (layer F.Cu) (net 2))
 (segment (start 196.58 186.42) (end 198.12 187.96) (width 0.254) (layer B.Cu) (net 2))
 (segment (start 193.675 186.42) (end 196.58 186.42) (width 0.254) (layer B.Cu) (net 2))
 (segment (start 188.0104 199.3396) (end 189.23 198.12) (width 0.254) (layer B.Cu) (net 2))
 (segment (start 188.0104 200.66) (end 188.0104 199.3396) (width 0.254) (layer B.Cu) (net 2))
 (segment (start 188.0104 201.1777) (end 188.0104 200.66) (width 0.254) (layer B.Cu) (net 2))
 (segment (start 188.7627 201.93) (end 188.0104 201.1777) (width 0.254) (layer B.Cu) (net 2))
 (segment (start 189.6863 201.93) (end 188.7627 201.93) (width 0.254) (layer B.Cu) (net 2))
 (segment (start 191.353 203.5967) (end 189.6863 201.93) (width 0.254) (layer B.Cu) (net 2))
 (segment (start 194.2897 200.66) (end 191.353 203.5967) (width 0.254) (layer B.Cu) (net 2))
 (segment (start 190.4641 207.6091) (end 191.77 208.915) (width 0.254) (layer B.Cu) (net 2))
 (segment (start 190.4641 204.4856) (end 190.4641 207.6091) (width 0.254) (layer B.Cu) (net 2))
 (segment (start 191.353 203.5967) (end 190.4641 204.4856) (width 0.254) (layer B.Cu) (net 2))
 (segment (start 190.8277 181.2823) (end 189.23 179.6847) (width 0.254) (layer F.Cu) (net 2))
 (segment (start 192.405 179.705) (end 190.8277 181.2823) (width 0.254) (layer F.Cu) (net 2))
 (segment (start 193.5941 186.42) (end 193.675 186.42) (width 0.254) (layer F.Cu) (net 2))
 (segment (start 190.8276 183.6535) (end 193.5941 186.42) (width 0.254) (layer F.Cu) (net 2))
 (segment (start 190.8276 181.2824) (end 190.8276 183.6535) (width 0.254) (layer F.Cu) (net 2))
 (segment (start 190.8277 181.2823) (end 190.8276 181.2824) (width 0.254) (layer F.Cu) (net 2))
 (segment (start 188.0104 200.66) (end 181.61 200.66) (width 0.254) (layer B.Cu) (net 2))
 (segment (start 176.5503 196.8703) (end 176.5503 198.12) (width 0.254) (layer F.Cu) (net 2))
 (segment (start 172.72 193.04) (end 176.5503 196.8703) (width 0.254) (layer F.Cu) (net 2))
 (segment (start 174.1452 191.6148) (end 174.1452 176.185) (width 0.254) (layer F.Cu) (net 2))
 (segment (start 172.72 193.04) (end 174.1452 191.6148) (width 0.254) (layer F.Cu) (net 2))
 (segment (start 179.145 176.185) (end 174.1452 176.185) (width 0.254) (layer F.Cu) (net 2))
 (segment (start 174.1452 176.185) (end 172.645 176.185) (width 0.254) (layer F.Cu) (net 2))
 (segment (start 180.3502 201.9198) (end 176.5503 198.12) (width 0.254) (layer F.Cu) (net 2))
 (segment (start 181.61 200.66) (end 180.3502 201.9198) (width 0.254) (layer F.Cu) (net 2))
 (segment (start 180.3502 201.9198) (end 177.8 204.47) (width 0.254) (layer F.Cu) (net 2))
 (segment (start 196.2439 210.1561) (end 198.12 208.28) (width 0.254) (layer B.Cu) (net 21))
 (segment (start 191.1061 210.1561) (end 196.2439 210.1561) (width 0.254) (layer B.Cu) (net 21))
 (segment (start 189.23 208.28) (end 191.1061 210.1561) (width 0.254) (layer B.Cu) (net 21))
 (segment (start 189.23 210.82) (end 198.12 210.82) (width 0.254) (layer B.Cu) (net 19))
 (segment (start 194.31 208.915) (end 194.31 205.74) (width 0.254) (layer F.Cu) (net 27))
 (segment (start 182.88 177.165) (end 181.61 177.165) (width 0.254) (layer B.Cu) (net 26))
 (segment (start 184.15 178.435) (end 182.88 177.165) (width 0.254) (layer B.Cu) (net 26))
 (segment (start 191.7903 200.66) (end 189.23 200.66) (width 0.254) (layer B.Cu) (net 30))
 (segment (start 179.03 205.74) (end 177.8 206.97) (width 0.254) (layer F.Cu) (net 28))
 (segment (start 181.61 205.74) (end 179.03 205.74) (width 0.254) (layer F.Cu) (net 28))
 (segment (start 179.03 203.2) (end 177.8 201.97) (width 0.254) (layer B.Cu) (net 29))
 (segment (start 181.61 203.2) (end 179.03 203.2) (width 0.254) (layer B.Cu) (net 29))
 (segment (start 195.7392 184.42) (end 193.675 184.42) (width 0.254) (layer B.Cu) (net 3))
 (segment (start 196.7392 185.42) (end 195.7392 184.42) (width 0.254) (layer B.Cu) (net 3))
 (segment (start 198.12 185.42) (end 196.7392 185.42) (width 0.254) (layer B.Cu) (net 3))
 (segment (start 193.4587 183.2987) (end 192.405 182.245) (width 0.254) (layer F.Cu) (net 3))
 (segment (start 193.675 183.2987) (end 193.4587 183.2987) (width 0.254) (layer F.Cu) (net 3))
 (segment (start 193.675 184.42) (end 193.675 183.2987) (width 0.254) (layer F.Cu) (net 3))
 (segment (start 195.5081 187.8881) (end 198.12 190.5) (width 0.254) (layer B.Cu) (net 4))
 (segment (start 193.5574 187.8881) (end 195.5081 187.8881) (width 0.254) (layer B.Cu) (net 4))
 (segment (start 192.5537 186.8844) (end 193.5574 187.8881) (width 0.254) (layer B.Cu) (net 4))
 (segment (start 192.5537 184.473) (end 192.5537 186.8844) (width 0.254) (layer B.Cu) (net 4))
 (segment (start 189.6905 181.6098) (end 192.5537 184.473) (width 0.254) (layer B.Cu) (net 4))
 (segment (start 184.0997 181.6098) (end 189.6905 181.6098) (width 0.254) (layer B.Cu) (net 4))
 (segment (start 182.8295 182.88) (end 184.0997 181.6098) (width 0.254) (layer B.Cu) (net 4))
 (segment (start 181.61 182.88) (end 182.8295 182.88) (width 0.254) (layer B.Cu) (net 4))
 (segment (start 181.61 182.88) (end 180.3905 182.88) (width 0.254) (layer F.Cu) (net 4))
 (segment (start 175.475 183.515) (end 172.645 180.685) (width 0.254) (layer B.Cu) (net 4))
 (segment (start 175.9153 183.515) (end 175.475 183.515) (width 0.254) (layer B.Cu) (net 4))
 (segment (start 177.165 184.7647) (end 176.3646 183.9643) (width 0.254) (layer F.Cu) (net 4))
 (segment (start 177.165 186.69) (end 177.165 184.7647) (width 0.254) (layer F.Cu) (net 4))
 (segment (start 176.3646 183.9643) (end 175.9153 183.515) (width 0.254) (layer F.Cu) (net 4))
 (segment (start 178.6944 181.6345) (end 179.145 181.6345) (width 0.254) (layer F.Cu) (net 4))
 (segment (start 176.3646 183.9643) (end 178.6944 181.6345) (width 0.254) (layer F.Cu) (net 4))
 (segment (start 180.3905 182.88) (end 179.145 181.6345) (width 0.254) (layer F.Cu) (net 4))
 (segment (start 179.145 181.6345) (end 179.145 180.685) (width 0.254) (layer F.Cu) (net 4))
 (segment (start 173.355 190.5) (end 172.72 190.5) (width 0.254) (layer B.Cu) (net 4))
 (segment (start 177.165 186.69) (end 173.355 190.5) (width 0.254) (layer B.Cu) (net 4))
 (via (at 187.4492 182.4556) (size 0.889) (layers F.Cu B.Cu) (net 5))
 (segment (start 175.3155 185.3645) (end 172.72 187.96) (width 0.254) (layer B.Cu) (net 5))
 (segment (start 177.7197 185.3645) (end 175.3155 185.3645) (width 0.254) (layer B.Cu) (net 5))
 (segment (start 180.0585 187.7033) (end 177.7197 185.3645) (width 0.254) (layer B.Cu) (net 5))
 (segment (start 180.0585 188.2036) (end 180.0585 187.7033) (width 0.254) (layer B.Cu) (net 5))
 (segment (start 181.0849 189.23) (end 180.0585 188.2036) (width 0.254) (layer B.Cu) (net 5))
 (segment (start 182.1067 189.23) (end 181.0849 189.23) (width 0.254) (layer B.Cu) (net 5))
 (segment (start 182.871 188.4657) (end 182.1067 189.23) (width 0.254) (layer B.Cu) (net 5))
 (segment (start 182.871 185.42) (end 182.871 188.4657) (width 0.254) (layer B.Cu) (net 5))
 (segment (start 181.61 185.42) (end 182.871 185.42) (width 0.254) (layer B.Cu) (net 5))
 (segment (start 184.4848 185.42) (end 187.4492 182.4556) (width 0.254) (layer B.Cu) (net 5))
 (segment (start 182.871 185.42) (end 184.4848 185.42) (width 0.254) (layer B.Cu) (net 5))
 (segment (start 187.9095 173.9395) (end 186.69 172.72) (width 0.254) (layer F.Cu) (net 5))
 (segment (start 187.9095 181.9953) (end 187.9095 173.9395) (width 0.254) (layer F.Cu) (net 5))
 (segment (start 187.4492 182.4556) (end 187.9095 181.9953) (width 0.254) (layer F.Cu) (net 5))
 (segment (start 189.23 205.74) (end 191.77 205.74) (width 0.254) (layer F.Cu) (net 22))
 (segment (start 196.8267 204.4467) (end 198.12 205.74) (width 0.254) (layer B.Cu) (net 22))
 (segment (start 193.0633 204.4467) (end 196.8267 204.4467) (width 0.254) (layer B.Cu) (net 22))
 (segment (start 191.77 205.74) (end 193.0633 204.4467) (width 0.254) (layer B.Cu) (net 22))
 (segment (start 187.8168 174.1332) (end 189.23 172.72) (width 0.254) (layer B.Cu) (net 6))
 (segment (start 179.1924 174.1332) (end 187.8168 174.1332) (width 0.254) (layer B.Cu) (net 6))
 (segment (start 177.2475 176.0781) (end 179.1924 174.1332) (width 0.254) (layer B.Cu) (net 6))
 (segment (start 177.2475 184.8351) (end 177.2475 176.0781) (width 0.254) (layer B.Cu) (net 6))
 (segment (start 178.4851 184.8351) (end 177.2475 184.8351) (width 0.254) (layer B.Cu) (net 6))
 (segment (start 181.61 187.96) (end 178.4851 184.8351) (width 0.254) (layer B.Cu) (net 6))
 (segment (start 173.3049 184.8351) (end 172.72 185.42) (width 0.254) (layer B.Cu) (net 6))
 (segment (start 177.2475 184.8351) (end 173.3049 184.8351) (width 0.254) (layer B.Cu) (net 6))
 (segment (start 179.0497 198.12) (end 181.61 198.12) (width 0.254) (layer B.Cu) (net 1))
 (segment (start 187.9803 178.435) (end 189.23 177.1853) (width 0.254) (layer B.Cu) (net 1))
 (segment (start 186.69 178.435) (end 187.9803 178.435) (width 0.254) (layer B.Cu) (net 1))
 (segment (start 194.675 174.895) (end 192.405 177.165) (width 0.254) (layer B.Cu) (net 1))
 (segment (start 196.215 174.895) (end 194.675 174.895) (width 0.254) (layer B.Cu) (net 1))
 (segment (start 179.0497 191.1147) (end 177.165 189.23) (width 0.254) (layer F.Cu) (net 1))
 (segment (start 179.0497 198.12) (end 179.0497 191.1147) (width 0.254) (layer F.Cu) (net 1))
 (segment (start 197.485 193.04) (end 198.12 193.04) (width 0.254) (layer B.Cu) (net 1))
 (segment (start 194.31 189.865) (end 197.485 193.04) (width 0.254) (layer B.Cu) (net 1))
 (segment (start 193.04 189.865) (end 194.31 189.865) (width 0.254) (layer F.Cu) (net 1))
 (segment (start 191.77 191.135) (end 193.04 189.865) (width 0.254) (layer F.Cu) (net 1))
 (segment (start 186.69 175.26) (end 186.69 178.435) (width 0.254) (layer F.Cu) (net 1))
 (segment (start 184.15 172.72) (end 186.69 175.26) (width 0.254) (layer F.Cu) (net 1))
 (segment (start 185.4201 199.3901) (end 185.4201 198.12) (width 0.254) (layer F.Cu) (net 1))
 (segment (start 189.23 203.2) (end 185.4201 199.3901) (width 0.254) (layer F.Cu) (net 1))
 (segment (start 185.4201 198.12) (end 181.61 198.12) (width 0.254) (layer F.Cu) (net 1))
 (segment (start 185.4201 192.5747) (end 188.7648 189.23) (width 0.254) (layer F.Cu) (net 1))
 (segment (start 185.4201 198.12) (end 185.4201 192.5747) (width 0.254) (layer F.Cu) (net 1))
 (segment (start 186.5986 187.0638) (end 188.7648 189.23) (width 0.254) (layer F.Cu) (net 1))
 (segment (start 186.5986 178.5264) (end 186.5986 187.0638) (width 0.254) (layer F.Cu) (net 1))
 (segment (start 186.69 178.435) (end 186.5986 178.5264) (width 0.254) (layer F.Cu) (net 1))
 (segment (start 189.865 189.23) (end 191.77 191.135) (width 0.254) (layer F.Cu) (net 1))
 (segment (start 188.7648 189.23) (end 189.865 189.23) (width 0.254) (layer F.Cu) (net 1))
 (segment (start 192.3847 177.1853) (end 192.405 177.165) (width 0.254) (layer F.Cu) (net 1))
 (segment (start 189.23 177.1853) (end 192.3847 177.1853) (width 0.254) (layer F.Cu) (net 1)))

